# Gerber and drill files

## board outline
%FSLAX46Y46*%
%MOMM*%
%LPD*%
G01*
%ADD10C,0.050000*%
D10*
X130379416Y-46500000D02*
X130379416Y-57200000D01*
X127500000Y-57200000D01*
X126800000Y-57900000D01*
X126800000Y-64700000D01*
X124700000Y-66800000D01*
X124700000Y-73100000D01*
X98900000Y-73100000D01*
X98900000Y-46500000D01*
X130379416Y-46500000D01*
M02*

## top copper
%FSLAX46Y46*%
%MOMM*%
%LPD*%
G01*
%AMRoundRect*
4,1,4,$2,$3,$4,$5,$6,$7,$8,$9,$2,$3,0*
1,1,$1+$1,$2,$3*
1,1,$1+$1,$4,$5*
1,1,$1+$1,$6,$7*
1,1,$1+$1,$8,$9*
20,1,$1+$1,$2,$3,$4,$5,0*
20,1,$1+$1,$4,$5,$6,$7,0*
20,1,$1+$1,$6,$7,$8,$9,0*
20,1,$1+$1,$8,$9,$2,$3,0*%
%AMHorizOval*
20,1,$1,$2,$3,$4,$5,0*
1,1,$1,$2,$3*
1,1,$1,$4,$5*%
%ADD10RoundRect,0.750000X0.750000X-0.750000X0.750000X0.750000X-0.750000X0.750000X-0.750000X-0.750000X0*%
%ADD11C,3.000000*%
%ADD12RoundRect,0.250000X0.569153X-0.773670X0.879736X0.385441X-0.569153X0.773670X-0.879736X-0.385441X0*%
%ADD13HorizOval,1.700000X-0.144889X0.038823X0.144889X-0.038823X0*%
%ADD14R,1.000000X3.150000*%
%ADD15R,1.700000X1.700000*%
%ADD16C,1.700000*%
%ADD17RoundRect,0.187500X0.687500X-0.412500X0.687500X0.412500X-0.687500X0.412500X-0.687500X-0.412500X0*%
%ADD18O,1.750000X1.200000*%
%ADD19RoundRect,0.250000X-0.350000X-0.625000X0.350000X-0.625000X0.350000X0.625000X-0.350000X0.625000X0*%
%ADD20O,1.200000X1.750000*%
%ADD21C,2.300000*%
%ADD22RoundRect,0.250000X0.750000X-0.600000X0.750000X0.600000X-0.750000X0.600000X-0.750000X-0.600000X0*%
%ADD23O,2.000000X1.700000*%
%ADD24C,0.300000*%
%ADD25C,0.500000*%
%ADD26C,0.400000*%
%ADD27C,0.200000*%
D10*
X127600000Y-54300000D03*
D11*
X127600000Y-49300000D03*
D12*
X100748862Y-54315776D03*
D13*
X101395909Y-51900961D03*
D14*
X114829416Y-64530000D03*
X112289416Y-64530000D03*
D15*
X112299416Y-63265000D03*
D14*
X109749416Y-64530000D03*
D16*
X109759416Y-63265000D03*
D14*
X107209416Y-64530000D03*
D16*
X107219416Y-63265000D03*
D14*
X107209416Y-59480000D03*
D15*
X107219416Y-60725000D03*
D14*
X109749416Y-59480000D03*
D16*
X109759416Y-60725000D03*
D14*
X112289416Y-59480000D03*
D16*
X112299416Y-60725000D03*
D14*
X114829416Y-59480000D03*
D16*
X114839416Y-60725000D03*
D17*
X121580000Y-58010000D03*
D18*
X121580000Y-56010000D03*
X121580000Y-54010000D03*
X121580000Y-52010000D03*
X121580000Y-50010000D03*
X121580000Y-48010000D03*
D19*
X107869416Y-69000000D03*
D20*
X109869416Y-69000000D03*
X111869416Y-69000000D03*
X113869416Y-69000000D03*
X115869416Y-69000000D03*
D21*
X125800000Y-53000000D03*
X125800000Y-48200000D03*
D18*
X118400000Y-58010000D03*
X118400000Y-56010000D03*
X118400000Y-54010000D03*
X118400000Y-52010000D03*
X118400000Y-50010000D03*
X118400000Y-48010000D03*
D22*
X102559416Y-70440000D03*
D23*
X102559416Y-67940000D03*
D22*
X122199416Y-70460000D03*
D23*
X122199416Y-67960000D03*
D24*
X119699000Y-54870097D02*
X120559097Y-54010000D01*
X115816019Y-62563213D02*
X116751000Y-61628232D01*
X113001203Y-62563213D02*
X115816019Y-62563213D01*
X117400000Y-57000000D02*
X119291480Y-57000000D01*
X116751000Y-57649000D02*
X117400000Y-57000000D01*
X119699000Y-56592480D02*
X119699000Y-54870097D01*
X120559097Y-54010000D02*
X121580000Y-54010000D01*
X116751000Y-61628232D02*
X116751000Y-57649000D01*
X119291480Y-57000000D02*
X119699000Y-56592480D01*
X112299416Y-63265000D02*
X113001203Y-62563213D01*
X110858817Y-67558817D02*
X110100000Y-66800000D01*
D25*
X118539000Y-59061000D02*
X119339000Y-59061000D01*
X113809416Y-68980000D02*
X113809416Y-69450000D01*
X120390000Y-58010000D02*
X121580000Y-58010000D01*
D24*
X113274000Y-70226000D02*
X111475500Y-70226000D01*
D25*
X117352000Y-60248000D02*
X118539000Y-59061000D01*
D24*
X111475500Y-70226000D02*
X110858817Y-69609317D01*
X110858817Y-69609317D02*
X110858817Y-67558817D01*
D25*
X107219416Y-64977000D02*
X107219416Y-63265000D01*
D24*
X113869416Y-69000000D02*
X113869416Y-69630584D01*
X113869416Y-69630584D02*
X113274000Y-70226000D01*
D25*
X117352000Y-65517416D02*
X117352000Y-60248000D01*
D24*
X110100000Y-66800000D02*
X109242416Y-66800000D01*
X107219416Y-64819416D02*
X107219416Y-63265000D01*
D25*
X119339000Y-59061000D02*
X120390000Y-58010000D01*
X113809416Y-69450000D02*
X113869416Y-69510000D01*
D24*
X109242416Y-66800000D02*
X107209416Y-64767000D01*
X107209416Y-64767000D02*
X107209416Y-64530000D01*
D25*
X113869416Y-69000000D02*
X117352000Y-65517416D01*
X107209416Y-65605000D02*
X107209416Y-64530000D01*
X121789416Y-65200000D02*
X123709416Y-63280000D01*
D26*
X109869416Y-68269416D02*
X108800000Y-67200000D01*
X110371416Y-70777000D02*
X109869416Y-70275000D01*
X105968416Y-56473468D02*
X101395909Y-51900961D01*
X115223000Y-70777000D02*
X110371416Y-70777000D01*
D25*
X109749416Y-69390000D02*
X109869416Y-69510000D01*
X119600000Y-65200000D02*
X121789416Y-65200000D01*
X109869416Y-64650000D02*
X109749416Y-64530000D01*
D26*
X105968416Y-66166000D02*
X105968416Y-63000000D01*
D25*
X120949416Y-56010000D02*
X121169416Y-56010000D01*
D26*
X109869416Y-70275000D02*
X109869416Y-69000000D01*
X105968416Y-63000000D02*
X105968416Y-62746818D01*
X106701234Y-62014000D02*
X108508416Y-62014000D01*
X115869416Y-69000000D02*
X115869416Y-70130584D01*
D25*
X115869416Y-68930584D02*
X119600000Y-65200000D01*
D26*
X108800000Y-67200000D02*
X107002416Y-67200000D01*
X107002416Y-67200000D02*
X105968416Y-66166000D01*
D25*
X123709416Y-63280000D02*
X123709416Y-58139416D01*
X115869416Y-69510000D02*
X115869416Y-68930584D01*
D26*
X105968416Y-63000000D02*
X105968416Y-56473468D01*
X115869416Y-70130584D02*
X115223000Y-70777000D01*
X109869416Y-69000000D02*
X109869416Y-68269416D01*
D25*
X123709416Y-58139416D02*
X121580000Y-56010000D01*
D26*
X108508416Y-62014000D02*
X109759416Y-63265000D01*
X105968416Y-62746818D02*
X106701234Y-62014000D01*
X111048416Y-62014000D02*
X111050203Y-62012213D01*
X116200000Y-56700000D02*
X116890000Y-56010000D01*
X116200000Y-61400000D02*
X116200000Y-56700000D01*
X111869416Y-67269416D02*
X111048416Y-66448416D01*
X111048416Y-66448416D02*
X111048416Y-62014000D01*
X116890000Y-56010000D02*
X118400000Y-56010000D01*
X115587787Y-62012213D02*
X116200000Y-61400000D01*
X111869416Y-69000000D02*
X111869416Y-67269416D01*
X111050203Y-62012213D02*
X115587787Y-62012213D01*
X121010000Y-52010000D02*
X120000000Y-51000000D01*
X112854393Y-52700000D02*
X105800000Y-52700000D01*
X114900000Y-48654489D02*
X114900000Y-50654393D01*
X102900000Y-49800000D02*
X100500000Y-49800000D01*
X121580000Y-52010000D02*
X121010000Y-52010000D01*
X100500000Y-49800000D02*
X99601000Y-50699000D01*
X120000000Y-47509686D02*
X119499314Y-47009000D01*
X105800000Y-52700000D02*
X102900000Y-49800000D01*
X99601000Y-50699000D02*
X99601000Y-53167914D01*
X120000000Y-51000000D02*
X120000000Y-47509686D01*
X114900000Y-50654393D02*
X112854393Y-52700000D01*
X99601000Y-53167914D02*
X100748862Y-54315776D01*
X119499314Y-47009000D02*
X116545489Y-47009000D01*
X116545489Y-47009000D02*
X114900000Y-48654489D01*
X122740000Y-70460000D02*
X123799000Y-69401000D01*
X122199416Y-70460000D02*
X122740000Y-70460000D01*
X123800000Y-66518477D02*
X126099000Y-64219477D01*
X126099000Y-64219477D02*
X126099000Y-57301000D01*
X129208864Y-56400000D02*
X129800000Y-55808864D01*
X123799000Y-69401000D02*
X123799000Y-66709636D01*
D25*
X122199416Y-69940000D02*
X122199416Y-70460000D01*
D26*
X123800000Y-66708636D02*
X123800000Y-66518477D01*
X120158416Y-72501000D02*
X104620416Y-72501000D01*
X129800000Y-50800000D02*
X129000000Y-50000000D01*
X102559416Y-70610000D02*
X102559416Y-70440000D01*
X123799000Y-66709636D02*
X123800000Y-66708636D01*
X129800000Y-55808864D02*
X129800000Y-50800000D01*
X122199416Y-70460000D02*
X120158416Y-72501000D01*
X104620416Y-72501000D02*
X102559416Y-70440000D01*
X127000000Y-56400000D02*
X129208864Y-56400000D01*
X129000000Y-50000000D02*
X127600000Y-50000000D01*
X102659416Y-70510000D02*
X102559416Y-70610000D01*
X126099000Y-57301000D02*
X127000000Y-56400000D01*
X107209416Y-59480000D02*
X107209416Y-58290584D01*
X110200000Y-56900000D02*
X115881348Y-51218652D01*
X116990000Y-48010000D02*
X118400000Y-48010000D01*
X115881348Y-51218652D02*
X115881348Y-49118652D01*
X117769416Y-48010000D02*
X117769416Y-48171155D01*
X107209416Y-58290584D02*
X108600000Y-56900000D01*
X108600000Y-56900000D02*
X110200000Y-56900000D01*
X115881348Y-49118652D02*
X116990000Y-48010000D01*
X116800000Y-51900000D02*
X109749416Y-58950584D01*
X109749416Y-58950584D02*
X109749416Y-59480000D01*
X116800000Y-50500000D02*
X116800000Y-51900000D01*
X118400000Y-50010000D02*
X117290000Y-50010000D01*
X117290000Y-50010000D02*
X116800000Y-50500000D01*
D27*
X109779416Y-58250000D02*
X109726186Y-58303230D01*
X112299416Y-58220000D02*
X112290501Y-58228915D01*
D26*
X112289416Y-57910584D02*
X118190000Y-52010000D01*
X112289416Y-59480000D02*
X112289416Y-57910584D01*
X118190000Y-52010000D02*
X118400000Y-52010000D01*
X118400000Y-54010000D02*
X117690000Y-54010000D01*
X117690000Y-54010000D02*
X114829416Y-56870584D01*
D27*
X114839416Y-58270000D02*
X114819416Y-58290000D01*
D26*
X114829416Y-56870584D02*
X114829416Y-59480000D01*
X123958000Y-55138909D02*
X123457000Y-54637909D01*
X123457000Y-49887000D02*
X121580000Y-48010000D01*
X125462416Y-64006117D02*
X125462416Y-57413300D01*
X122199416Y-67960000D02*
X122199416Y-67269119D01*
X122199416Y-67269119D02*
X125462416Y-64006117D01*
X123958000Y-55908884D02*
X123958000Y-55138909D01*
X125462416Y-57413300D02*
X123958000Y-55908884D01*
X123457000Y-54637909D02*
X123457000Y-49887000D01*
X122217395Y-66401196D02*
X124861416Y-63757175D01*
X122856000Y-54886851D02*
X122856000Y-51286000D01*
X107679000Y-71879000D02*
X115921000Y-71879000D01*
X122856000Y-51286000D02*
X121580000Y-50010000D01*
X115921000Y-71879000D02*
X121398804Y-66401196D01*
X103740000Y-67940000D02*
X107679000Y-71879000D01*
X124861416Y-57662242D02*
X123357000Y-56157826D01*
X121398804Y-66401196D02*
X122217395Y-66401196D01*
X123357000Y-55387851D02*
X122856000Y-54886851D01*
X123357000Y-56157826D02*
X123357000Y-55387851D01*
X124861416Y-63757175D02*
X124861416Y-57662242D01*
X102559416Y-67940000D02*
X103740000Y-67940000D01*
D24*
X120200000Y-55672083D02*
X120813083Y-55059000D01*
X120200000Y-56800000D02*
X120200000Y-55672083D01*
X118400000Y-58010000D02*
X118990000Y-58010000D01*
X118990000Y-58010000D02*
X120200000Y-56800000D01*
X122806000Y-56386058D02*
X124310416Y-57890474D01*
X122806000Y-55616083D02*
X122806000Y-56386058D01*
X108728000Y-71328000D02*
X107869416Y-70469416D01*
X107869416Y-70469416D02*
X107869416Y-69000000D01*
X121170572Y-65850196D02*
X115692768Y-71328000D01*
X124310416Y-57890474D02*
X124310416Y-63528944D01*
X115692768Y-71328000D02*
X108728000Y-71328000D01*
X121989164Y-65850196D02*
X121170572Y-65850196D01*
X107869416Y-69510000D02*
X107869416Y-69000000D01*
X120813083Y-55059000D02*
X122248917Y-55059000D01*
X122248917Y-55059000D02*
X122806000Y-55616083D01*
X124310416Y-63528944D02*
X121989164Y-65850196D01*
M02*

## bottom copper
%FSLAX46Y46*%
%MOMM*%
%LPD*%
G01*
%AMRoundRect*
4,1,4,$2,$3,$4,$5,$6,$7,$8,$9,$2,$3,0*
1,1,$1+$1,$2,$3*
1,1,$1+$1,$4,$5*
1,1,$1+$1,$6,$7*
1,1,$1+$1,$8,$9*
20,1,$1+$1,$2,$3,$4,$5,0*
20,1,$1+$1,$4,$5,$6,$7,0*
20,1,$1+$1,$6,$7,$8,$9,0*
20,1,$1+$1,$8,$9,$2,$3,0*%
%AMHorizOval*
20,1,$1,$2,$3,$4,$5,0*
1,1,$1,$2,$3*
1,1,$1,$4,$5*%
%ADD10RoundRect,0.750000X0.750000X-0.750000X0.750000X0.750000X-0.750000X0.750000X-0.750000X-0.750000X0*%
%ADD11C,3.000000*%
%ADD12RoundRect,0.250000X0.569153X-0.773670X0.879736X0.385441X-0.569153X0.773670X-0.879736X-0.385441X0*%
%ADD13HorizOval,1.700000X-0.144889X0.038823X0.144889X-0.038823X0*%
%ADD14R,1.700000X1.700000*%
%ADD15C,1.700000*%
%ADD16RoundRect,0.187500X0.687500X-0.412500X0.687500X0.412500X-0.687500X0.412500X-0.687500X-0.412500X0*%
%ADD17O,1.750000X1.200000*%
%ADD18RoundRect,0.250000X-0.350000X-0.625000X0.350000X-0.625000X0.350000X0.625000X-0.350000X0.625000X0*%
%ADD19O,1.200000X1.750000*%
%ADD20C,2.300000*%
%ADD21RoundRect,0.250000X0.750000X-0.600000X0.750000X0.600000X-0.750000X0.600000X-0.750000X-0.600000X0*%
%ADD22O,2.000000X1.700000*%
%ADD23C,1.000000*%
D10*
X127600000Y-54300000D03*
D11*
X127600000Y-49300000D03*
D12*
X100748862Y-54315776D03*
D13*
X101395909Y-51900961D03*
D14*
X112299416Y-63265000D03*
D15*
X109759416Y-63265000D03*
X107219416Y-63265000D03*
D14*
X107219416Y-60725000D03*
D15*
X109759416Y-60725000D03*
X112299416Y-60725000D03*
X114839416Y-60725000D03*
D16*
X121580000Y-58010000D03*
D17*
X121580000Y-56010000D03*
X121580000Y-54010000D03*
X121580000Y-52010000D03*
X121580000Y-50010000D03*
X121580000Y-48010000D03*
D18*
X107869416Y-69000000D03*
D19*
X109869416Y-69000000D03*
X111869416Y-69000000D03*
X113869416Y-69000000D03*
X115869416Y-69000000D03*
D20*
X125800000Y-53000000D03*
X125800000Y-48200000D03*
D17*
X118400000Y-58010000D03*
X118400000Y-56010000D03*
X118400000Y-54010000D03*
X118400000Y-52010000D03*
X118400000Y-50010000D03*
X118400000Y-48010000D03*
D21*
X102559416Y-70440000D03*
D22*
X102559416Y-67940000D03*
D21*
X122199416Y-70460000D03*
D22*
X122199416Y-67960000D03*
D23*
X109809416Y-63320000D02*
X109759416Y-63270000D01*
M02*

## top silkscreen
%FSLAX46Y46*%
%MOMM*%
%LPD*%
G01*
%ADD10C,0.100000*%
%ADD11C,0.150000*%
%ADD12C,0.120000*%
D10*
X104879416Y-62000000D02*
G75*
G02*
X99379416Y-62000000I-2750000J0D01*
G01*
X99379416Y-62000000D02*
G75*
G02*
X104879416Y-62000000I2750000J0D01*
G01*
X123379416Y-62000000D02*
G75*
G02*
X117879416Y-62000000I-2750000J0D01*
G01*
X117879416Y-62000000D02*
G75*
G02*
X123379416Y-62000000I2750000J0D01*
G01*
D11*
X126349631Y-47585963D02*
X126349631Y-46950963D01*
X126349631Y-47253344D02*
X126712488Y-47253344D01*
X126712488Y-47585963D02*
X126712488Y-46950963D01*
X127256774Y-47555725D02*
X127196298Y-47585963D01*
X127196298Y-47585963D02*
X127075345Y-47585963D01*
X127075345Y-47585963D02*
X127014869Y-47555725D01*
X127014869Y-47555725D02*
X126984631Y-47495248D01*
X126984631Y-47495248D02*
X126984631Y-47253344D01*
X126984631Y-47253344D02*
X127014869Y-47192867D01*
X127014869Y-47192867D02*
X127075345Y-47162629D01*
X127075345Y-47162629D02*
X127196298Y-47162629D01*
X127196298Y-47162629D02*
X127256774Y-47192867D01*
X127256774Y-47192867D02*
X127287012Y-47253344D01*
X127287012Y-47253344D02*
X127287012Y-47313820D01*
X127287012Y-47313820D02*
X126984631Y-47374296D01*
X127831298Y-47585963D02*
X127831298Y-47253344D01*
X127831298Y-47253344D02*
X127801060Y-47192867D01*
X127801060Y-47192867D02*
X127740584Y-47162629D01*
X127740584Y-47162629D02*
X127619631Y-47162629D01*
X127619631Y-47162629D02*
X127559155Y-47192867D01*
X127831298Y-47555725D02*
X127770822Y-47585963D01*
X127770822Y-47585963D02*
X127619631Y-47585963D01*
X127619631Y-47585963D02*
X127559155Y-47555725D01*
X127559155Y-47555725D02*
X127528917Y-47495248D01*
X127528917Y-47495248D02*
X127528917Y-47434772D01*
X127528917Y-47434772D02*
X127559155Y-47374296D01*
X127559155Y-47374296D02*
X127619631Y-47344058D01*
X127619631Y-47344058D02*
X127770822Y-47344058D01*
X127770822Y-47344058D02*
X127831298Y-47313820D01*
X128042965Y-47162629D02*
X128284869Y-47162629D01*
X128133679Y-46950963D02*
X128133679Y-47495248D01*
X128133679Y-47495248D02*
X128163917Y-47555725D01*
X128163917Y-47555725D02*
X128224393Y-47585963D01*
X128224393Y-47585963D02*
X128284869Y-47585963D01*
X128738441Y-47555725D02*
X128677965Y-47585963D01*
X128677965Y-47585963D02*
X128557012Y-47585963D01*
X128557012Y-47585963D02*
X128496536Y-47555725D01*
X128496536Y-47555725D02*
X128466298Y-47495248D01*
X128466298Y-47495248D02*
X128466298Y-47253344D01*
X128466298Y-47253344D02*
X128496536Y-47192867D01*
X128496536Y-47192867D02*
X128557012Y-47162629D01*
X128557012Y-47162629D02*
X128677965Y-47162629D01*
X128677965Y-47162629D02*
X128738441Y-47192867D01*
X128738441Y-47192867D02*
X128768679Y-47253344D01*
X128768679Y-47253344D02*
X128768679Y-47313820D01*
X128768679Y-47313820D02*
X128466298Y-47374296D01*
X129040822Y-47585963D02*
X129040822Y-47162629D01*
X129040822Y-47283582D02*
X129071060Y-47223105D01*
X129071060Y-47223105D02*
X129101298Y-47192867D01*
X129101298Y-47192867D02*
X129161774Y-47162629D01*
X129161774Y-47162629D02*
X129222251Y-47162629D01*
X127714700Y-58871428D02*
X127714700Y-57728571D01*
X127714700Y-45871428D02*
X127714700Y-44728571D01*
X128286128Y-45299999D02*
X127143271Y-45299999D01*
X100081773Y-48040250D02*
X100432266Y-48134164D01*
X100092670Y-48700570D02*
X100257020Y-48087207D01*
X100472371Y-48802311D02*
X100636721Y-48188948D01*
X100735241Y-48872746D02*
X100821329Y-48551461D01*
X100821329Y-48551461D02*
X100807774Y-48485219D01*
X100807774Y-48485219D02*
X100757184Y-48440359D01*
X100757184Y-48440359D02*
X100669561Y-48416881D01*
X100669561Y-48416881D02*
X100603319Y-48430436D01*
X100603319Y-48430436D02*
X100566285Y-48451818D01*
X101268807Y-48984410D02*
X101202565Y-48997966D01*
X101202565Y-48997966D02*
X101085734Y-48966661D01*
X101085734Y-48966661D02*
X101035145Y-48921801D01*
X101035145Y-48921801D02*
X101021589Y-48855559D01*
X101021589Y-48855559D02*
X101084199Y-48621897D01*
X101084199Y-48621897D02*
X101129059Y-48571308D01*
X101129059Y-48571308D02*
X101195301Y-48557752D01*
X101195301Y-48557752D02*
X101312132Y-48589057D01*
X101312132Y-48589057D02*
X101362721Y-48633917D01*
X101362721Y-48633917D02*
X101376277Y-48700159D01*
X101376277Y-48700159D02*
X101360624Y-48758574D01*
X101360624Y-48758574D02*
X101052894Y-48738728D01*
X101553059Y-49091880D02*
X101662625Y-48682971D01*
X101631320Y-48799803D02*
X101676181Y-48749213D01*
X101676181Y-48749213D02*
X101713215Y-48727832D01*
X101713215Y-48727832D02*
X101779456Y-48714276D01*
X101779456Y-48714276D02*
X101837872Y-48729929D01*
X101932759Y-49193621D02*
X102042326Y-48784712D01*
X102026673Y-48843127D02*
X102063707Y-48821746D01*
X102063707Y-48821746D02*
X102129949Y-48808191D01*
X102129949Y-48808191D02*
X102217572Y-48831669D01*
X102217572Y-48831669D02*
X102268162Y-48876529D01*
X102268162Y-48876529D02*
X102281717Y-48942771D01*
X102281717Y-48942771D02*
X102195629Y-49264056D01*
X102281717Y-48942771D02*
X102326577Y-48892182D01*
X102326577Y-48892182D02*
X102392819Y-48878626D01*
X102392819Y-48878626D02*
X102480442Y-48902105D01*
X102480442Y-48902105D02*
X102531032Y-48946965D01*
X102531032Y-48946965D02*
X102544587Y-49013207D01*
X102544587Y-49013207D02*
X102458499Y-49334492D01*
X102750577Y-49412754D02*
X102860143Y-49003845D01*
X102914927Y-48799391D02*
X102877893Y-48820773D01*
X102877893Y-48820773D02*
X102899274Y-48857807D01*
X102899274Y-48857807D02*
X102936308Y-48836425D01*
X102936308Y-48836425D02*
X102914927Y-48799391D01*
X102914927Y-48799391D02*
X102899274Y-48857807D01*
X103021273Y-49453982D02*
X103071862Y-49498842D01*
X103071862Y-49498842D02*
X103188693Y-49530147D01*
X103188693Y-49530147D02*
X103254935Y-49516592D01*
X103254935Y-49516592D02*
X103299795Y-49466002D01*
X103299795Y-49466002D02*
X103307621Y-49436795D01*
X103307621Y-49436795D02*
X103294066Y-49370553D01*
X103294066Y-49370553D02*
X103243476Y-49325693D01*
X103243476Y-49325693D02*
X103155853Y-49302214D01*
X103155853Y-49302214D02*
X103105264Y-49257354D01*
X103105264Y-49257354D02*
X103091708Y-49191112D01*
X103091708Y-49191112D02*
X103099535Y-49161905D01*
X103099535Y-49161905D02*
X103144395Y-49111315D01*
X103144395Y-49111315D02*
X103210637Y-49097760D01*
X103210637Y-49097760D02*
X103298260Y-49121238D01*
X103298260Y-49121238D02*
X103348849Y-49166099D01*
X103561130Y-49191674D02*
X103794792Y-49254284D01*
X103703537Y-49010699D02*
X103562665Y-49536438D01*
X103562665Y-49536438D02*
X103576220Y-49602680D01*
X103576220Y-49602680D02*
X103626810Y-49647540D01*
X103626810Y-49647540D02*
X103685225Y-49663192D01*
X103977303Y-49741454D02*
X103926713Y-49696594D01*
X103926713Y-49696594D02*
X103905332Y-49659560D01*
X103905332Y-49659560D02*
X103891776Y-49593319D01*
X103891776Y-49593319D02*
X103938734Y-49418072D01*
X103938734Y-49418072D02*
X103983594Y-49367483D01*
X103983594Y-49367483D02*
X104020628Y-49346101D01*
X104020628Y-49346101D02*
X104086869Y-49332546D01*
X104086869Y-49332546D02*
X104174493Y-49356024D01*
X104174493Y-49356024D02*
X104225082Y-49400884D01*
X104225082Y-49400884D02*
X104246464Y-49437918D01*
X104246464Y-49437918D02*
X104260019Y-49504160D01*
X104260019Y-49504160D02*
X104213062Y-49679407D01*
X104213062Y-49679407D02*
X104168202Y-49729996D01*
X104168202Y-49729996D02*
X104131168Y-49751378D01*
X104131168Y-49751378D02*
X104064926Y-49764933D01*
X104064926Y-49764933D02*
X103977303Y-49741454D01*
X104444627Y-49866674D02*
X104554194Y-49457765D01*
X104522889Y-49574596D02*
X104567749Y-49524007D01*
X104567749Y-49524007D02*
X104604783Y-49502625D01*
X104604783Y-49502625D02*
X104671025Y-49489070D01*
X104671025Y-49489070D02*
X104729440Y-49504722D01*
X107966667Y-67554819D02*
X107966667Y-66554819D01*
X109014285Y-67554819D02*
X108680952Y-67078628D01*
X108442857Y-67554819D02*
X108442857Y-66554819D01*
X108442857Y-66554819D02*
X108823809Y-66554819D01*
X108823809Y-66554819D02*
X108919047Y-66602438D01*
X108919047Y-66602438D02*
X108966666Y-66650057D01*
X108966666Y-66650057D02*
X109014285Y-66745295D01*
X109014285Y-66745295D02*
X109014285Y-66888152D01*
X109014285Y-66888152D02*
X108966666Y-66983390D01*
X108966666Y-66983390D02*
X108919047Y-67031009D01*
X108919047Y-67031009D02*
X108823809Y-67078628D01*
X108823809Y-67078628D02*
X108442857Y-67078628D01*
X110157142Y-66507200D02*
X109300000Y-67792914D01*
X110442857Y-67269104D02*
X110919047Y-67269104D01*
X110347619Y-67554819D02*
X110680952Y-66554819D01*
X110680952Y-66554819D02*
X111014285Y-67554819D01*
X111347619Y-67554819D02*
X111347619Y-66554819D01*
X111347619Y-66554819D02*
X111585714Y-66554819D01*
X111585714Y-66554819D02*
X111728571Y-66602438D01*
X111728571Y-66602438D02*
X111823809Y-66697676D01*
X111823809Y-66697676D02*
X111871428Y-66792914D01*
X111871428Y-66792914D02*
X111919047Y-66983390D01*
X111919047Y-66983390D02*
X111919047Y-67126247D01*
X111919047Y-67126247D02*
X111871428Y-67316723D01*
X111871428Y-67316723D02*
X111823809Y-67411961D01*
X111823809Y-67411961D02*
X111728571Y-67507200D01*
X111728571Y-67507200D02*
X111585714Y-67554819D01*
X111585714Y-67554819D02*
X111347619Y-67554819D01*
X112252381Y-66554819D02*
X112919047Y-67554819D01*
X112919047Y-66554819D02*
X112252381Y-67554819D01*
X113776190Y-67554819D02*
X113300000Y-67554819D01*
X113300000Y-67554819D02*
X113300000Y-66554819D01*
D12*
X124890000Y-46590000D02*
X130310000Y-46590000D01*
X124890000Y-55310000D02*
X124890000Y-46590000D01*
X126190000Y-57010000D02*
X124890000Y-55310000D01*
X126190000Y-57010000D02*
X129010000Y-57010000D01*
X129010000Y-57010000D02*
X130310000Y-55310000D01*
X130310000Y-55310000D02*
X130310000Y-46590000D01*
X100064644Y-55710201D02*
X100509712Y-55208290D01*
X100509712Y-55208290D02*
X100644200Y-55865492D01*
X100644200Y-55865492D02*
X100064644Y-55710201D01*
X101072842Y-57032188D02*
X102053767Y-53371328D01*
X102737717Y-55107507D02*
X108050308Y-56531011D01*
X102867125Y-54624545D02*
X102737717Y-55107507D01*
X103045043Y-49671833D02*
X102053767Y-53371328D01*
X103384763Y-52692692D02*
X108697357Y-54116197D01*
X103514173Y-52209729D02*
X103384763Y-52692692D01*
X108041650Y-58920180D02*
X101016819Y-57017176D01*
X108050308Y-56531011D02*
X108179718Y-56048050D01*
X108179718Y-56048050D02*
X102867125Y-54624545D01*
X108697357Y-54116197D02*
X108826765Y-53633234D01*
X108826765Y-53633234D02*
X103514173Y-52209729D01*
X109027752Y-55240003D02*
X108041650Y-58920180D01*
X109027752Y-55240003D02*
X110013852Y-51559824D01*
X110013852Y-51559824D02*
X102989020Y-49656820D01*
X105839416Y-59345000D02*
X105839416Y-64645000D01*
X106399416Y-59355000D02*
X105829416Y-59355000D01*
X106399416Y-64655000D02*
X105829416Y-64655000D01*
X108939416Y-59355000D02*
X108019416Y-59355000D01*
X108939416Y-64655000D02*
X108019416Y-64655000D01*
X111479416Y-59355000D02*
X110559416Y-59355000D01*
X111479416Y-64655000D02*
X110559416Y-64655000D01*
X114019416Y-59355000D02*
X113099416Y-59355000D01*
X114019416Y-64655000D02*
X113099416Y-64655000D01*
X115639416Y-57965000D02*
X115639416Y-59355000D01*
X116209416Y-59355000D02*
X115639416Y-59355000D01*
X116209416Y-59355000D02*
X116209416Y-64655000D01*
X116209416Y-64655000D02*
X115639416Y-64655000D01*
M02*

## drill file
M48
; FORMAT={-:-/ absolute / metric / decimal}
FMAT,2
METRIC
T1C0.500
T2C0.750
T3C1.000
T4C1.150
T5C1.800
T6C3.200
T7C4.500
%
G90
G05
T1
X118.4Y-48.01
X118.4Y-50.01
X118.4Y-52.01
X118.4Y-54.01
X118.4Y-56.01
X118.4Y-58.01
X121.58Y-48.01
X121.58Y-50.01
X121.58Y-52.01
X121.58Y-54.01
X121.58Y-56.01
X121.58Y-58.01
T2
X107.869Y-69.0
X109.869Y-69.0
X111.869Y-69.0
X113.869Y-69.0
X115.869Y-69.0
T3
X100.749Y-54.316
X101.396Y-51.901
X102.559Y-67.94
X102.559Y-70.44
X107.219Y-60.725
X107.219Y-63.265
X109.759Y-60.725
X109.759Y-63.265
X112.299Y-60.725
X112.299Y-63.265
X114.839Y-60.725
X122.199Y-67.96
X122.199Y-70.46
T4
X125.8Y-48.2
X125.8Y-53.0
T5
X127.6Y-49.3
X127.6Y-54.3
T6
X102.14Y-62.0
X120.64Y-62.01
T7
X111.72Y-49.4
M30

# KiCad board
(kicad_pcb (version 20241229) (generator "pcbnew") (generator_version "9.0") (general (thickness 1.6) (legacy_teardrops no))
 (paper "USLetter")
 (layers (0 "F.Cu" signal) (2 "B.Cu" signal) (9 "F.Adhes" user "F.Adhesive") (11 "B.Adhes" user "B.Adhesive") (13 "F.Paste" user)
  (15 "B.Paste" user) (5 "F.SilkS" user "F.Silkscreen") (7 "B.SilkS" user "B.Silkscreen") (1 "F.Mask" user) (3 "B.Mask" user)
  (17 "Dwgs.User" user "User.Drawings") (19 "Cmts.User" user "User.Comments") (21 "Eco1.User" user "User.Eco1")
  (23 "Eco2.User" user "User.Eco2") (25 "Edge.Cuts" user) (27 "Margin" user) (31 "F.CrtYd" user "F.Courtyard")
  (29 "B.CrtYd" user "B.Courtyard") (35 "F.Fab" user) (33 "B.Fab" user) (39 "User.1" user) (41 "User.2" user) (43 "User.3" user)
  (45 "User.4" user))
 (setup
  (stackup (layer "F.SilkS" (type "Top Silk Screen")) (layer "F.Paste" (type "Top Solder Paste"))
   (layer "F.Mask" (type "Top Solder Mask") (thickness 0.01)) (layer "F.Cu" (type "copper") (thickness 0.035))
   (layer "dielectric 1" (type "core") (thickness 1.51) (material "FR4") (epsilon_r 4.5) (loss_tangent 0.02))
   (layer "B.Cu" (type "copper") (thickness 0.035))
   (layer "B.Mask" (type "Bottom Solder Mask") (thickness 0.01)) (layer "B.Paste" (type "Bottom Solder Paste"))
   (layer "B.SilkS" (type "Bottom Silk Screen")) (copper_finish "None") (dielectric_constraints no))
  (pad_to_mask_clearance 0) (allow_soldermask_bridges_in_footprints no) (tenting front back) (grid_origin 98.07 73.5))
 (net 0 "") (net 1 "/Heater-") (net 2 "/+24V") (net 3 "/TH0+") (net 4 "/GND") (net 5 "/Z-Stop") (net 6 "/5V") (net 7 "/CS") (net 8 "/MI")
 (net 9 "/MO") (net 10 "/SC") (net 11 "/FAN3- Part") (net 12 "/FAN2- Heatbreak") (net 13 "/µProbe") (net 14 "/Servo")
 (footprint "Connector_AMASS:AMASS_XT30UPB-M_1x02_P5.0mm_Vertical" (layer "F.Cu") (at 127.6 54.3 90)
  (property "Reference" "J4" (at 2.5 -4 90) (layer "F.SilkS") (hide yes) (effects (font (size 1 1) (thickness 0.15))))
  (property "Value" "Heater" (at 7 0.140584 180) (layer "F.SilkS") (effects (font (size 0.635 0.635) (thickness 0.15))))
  (fp_line (start 7.71 -2.71) (end 7.71 2.71) (stroke (width 0.12) (type solid)) (layer "F.SilkS"))
  (fp_line (start -1.01 -2.71) (end 7.71 -2.71) (stroke (width 0.12) (type solid)) (layer "F.SilkS"))
  (fp_line (start -2.71 -1.41) (end -1.01 -2.71) (stroke (width 0.12) (type solid)) (layer "F.SilkS"))
  (fp_line (start -2.71 -1.41) (end -2.71 1.41) (stroke (width 0.12) (type solid)) (layer "F.SilkS"))
  (fp_line (start -2.71 1.41) (end -1.01 2.71) (stroke (width 0.12) (type solid)) (layer "F.SilkS"))
  (fp_line (start -1.01 2.71) (end 7.71 2.71) (stroke (width 0.12) (type solid)) (layer "F.SilkS"))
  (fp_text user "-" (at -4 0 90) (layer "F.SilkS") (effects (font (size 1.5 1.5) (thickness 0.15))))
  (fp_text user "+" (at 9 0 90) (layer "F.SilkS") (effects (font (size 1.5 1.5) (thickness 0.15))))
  (pad "1" thru_hole roundrect (at 0 0 90) (size 3 3) (drill 1.8) (layers "*.Cu" "*.Mask") (remove_unused_layers no) (roundrect_rratio 0.25)
   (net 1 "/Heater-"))
  (pad "2" thru_hole circle (at 5 0 90) (size 3 3) (drill 1.8) (layers "*.Cu" "*.Mask") (remove_unused_layers no) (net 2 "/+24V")))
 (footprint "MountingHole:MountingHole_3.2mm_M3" (layer "F.Cu") (at 120.64 62.01)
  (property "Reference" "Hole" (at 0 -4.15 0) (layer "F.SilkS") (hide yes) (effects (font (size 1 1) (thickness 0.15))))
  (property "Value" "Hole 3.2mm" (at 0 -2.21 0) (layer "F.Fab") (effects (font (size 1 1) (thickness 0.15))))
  (pad "" np_thru_hole circle (at 0 0) (size 3.2 3.2) (drill 3.2) (layers "*.Cu" "*.Mask")))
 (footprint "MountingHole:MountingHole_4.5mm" (layer "F.Cu") (at 111.72 49.4)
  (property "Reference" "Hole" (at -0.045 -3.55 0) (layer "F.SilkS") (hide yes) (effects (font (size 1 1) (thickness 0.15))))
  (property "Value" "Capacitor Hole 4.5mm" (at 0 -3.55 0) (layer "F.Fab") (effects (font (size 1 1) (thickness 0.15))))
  (pad "" np_thru_hole circle (at 0 0) (size 4.5 4.5) (drill 4.5) (layers "*.Cu" "*.Mask")))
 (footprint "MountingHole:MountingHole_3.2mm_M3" (layer "F.Cu") (at 102.14 62)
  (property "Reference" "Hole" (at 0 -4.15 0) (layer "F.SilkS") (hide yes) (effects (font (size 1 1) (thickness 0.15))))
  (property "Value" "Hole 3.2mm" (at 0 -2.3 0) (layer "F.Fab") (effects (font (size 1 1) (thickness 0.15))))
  (pad "" np_thru_hole circle (at 0 0) (size 3.2 3.2) (drill 3.2) (layers "*.Cu" "*.Mask")))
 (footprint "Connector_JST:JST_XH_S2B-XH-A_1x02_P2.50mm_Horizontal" (layer "F.Cu") (at 100.748862 54.315776 75)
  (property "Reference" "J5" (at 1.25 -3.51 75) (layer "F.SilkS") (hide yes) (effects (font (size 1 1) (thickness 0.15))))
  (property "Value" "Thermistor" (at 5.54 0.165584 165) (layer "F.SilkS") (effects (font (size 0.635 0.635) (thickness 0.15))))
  (fp_line (start -1.524 -0.3) (end -0.923999 -0.000002) (stroke (width 0.12) (type solid)) (layer "F.SilkS"))
  (fp_line (start -0.923999 -0.000002) (end -1.523999 0.3) (stroke (width 0.12) (type solid)) (layer "F.SilkS"))
  (fp_line (start -1.523999 0.3) (end -1.524 -0.3) (stroke (width 0.12) (type solid)) (layer "F.SilkS"))
  (fp_line (start -2.54 1.016) (end 1.250001 1.016) (stroke (width 0.12) (type solid)) (layer "F.SilkS"))
  (fp_line (start -0.25 2.126001) (end -0.249999 7.626) (stroke (width 0.12) (type solid)) (layer "F.SilkS"))
  (fp_line (start 0.249999 2.126) (end -0.25 2.126001) (stroke (width 0.12) (type solid)) (layer "F.SilkS"))
  (fp_line (start 5.08 1.016) (end 1.250001 1.016) (stroke (width 0.12) (type solid)) (layer "F.SilkS"))
  (fp_line (start 2.25 2.126) (end 2.25 7.626002) (stroke (width 0.12) (type solid)) (layer "F.SilkS"))
  (fp_line (start 2.75 2.126) (end 2.25 2.126) (stroke (width 0.12) (type solid)) (layer "F.SilkS"))
  (fp_line (start -2.56 8.236) (end -2.54 0.958) (stroke (width 0.12) (type solid)) (layer "F.SilkS"))
  (fp_line (start -0.249999 7.626) (end 0.249999 7.626001) (stroke (width 0.12) (type solid)) (layer "F.SilkS"))
  (fp_line (start 0.249999 7.626001) (end 0.249999 2.126) (stroke (width 0.12) (type solid)) (layer "F.SilkS"))
  (fp_line (start 2.25 7.626002) (end 2.75 7.626) (stroke (width 0.12) (type solid)) (layer "F.SilkS"))
  (fp_line (start 2.75 7.626) (end 2.75 2.126) (stroke (width 0.12) (type solid)) (layer "F.SilkS"))
  (fp_line (start 1.25 8.236001) (end -2.56 8.236) (stroke (width 0.12) (type solid)) (layer "F.SilkS"))
  (fp_line (start 1.25 8.236001) (end 5.060001 8.236) (stroke (width 0.12) (type solid)) (layer "F.SilkS"))
  (fp_line (start 5.060001 8.236) (end 5.080001 0.958) (stroke (width 0.12) (type solid)) (layer "F.SilkS"))
  (pad "1" thru_hole roundrect (at 0 0 75) (size 1.7 2) (drill 1) (layers "*.Cu" "*.Mask") (remove_unused_layers no)
   (roundrect_rratio 0.147059) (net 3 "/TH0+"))
  (pad "2" thru_hole oval (at 2.5 -0.000001 75) (size 1.7 2) (drill 1) (layers "*.Cu" "*.Mask") (remove_unused_layers no) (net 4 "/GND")))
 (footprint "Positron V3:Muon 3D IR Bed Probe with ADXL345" (layer "F.Cu") (at 109.339416 58.225)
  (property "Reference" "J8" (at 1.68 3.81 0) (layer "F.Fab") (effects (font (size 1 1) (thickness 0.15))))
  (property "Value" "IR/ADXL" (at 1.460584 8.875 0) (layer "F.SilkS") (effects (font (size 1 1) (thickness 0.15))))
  (fp_line (start -3.5 1.12) (end -3.5 6.42) (stroke (width 0.12) (type solid)) (layer "F.SilkS"))
  (fp_line (start -2.94 1.13) (end -3.51 1.13) (stroke (width 0.12) (type solid)) (layer "F.SilkS"))
  (fp_line (start -2.94 6.43) (end -3.51 6.43) (stroke (width 0.12) (type solid)) (layer "F.SilkS"))
  (fp_line (start -0.4 1.13) (end -1.32 1.13) (stroke (width 0.12) (type solid)) (layer "F.SilkS"))
  (fp_line (start -0.4 6.43) (end -1.32 6.43) (stroke (width 0.12) (type solid)) (layer "F.SilkS"))
  (fp_line (start 2.14 1.13) (end 1.22 1.13) (stroke (width 0.12) (type solid)) (layer "F.SilkS"))
  (fp_line (start 2.14 6.43) (end 1.22 6.43) (stroke (width 0.12) (type solid)) (layer "F.SilkS"))
  (fp_line (start 4.68 1.13) (end 3.76 1.13) (stroke (width 0.12) (type solid)) (layer "F.SilkS"))
  (fp_line (start 4.68 6.43) (end 3.76 6.43) (stroke (width 0.12) (type solid)) (layer "F.SilkS"))
  (fp_line (start 6.3 -0.26) (end 6.3 1.13) (stroke (width 0.12) (type solid)) (layer "F.SilkS"))
  (fp_line (start 6.87 1.13) (end 6.3 1.13) (stroke (width 0.12) (type solid)) (layer "F.SilkS"))
  (fp_line (start 6.87 1.13) (end 6.87 6.43) (stroke (width 0.12) (type solid)) (layer "F.SilkS"))
  (fp_line (start 6.87 6.43) (end 6.3 6.43) (stroke (width 0.12) (type solid)) (layer "F.SilkS"))
  (pad "" smd rect (at 5.49 6.305 270) (size 3.15 1) (layers "F.Cu" "F.Mask" "F.Paste"))
  (pad "1" smd rect (at 2.95 6.305 270) (size 3.15 1) (layers "F.Cu" "F.Mask" "F.Paste") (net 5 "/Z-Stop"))
  (pad "1" thru_hole rect (at 2.96 5.04 270) (size 1.7 1.7) (drill 1) (layers "*.Cu" "*.Mask") (remove_unused_layers no) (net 5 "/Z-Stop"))
  (pad "2" smd rect (at 0.41 6.305 270) (size 3.15 1) (layers "F.Cu" "F.Mask" "F.Paste") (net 4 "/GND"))
  (pad "2" thru_hole circle (at 0.42 5.04 270) (size 1.7 1.7) (drill 1) (layers "*.Cu" "*.Mask") (remove_unused_layers no) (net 4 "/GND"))
  (pad "3" smd rect (at -2.13 6.305 270) (size 3.15 1) (layers "F.Cu" "F.Mask" "F.Paste") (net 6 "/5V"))
  (pad "3" thru_hole circle (at -2.12 5.04 270) (size 1.7 1.7) (drill 1) (layers "*.Cu" "*.Mask") (remove_unused_layers no) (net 6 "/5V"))
  (pad "4" smd rect (at -2.13 1.255 270) (size 3.15 1) (layers "F.Cu" "F.Mask" "F.Paste") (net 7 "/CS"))
  (pad "4" thru_hole rect (at -2.12 2.5 270) (size 1.7 1.7) (drill 1) (layers "*.Cu" "*.Mask") (remove_unused_layers no) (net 7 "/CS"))
  (pad "5" smd rect (at 0.41 1.255 270) (size 3.15 1) (layers "F.Cu" "F.Mask" "F.Paste") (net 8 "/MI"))
  (pad "5" thru_hole circle (at 0.42 2.5 270) (size 1.7 1.7) (drill 1) (layers "*.Cu" "*.Mask") (remove_unused_layers no) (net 8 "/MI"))
  (pad "6" smd rect (at 2.95 1.255 270) (size 3.15 1) (layers "F.Cu" "F.Mask" "F.Paste") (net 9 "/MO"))
  (pad "6" thru_hole circle (at 2.96 2.5 270) (size 1.7 1.7) (drill 1) (layers "*.Cu" "*.Mask") (remove_unused_layers no) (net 9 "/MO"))
  (pad "7" smd rect (at 5.49 1.255 270) (size 3.15 1) (layers "F.Cu" "F.Mask" "F.Paste") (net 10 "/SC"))
  (pad "7" thru_hole circle (at 5.5 2.5 270) (size 1.7 1.7) (drill 1) (layers "*.Cu" "*.Mask") (remove_unused_layers no) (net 10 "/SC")))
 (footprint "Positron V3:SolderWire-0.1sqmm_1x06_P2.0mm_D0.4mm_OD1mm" (layer "B.Cu") (at 121.58 58.01 90)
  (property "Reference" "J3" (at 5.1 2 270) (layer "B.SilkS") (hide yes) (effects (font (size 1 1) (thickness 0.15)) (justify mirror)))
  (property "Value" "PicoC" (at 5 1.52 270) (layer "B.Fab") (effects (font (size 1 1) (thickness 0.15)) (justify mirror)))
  (pad "1" thru_hole roundrect (at 0 0 90) (size 1.2 1.75) (drill 0.5) (layers "*.Cu" "*.Mask") (remove_unused_layers no)
   (roundrect_rratio 0.15625) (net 6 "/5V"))
  (pad "2" thru_hole oval (at 2 0 90) (size 1.2 1.75) (drill 0.5) (layers "*.Cu" "*.Mask") (remove_unused_layers no) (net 4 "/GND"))
  (pad "3" thru_hole oval (at 4 0 90) (size 1.2 1.75) (drill 0.5) (layers "*.Cu" "*.Mask") (remove_unused_layers no) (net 5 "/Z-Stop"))
  (pad "4" thru_hole oval (at 6 0 90) (size 1.2 1.75) (drill 0.5) (layers "*.Cu" "*.Mask") (remove_unused_layers no) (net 3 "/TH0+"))
  (pad "5" thru_hole oval (at 8 0 90) (size 1.2 1.75) (drill 0.5) (layers "*.Cu" "*.Mask") (remove_unused_layers no) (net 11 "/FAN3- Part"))
  (pad "6" thru_hole oval (at 10 0 90) (size 1.2 1.75) (drill 0.5) (layers "*.Cu" "*.Mask") (remove_unused_layers no)
   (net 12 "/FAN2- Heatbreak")))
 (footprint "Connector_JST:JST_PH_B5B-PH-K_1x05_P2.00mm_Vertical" (layer "B.Cu") (at 107.869416 69)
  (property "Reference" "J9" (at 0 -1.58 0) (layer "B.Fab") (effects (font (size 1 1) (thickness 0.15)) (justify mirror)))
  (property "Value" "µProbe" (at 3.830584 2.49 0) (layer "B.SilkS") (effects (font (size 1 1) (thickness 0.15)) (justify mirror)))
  (pad "1" thru_hole roundrect (at 0 0) (size 1.2 1.75) (drill 0.75) (layers "*.Cu" "*.Mask") (remove_unused_layers no)
   (roundrect_rratio 0.208333) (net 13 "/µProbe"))
  (pad "2" thru_hole oval (at 2 0) (size 1.2 1.75) (drill 0.75) (layers "*.Cu" "*.Mask") (remove_unused_layers no) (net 4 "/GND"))
  (pad "3" thru_hole oval (at 4 0) (size 1.2 1.75) (drill 0.75) (layers "*.Cu" "*.Mask") (remove_unused_layers no) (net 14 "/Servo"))
  (pad "4" thru_hole oval (at 6 0) (size 1.2 1.75) (drill 0.75) (layers "*.Cu" "*.Mask") (remove_unused_layers no) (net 6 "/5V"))
  (pad "5" thru_hole oval (at 8 0) (size 1.2 1.75) (drill 0.75) (layers "*.Cu" "*.Mask") (remove_unused_layers no) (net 4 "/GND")))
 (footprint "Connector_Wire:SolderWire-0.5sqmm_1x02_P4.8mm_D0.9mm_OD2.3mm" (layer "B.Cu") (at 125.8 53 90)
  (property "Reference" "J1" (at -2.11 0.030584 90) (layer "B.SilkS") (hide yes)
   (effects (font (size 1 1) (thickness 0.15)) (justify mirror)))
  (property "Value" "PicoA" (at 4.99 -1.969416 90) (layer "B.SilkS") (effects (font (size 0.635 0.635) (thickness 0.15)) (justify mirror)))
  (pad "1" thru_hole circle (at 0 0 90) (size 2.3 2.3) (drill 1.15) (layers "*.Cu" "*.Mask") (remove_unused_layers no) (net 1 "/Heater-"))
  (pad "2" thru_hole circle (at 4.8 0 90) (size 2.3 2.3) (drill 1.15) (layers "*.Cu" "*.Mask") (remove_unused_layers no) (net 2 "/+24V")))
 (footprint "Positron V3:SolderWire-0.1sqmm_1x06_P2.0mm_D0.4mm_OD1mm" (layer "B.Cu") (at 118.4 58.01 90)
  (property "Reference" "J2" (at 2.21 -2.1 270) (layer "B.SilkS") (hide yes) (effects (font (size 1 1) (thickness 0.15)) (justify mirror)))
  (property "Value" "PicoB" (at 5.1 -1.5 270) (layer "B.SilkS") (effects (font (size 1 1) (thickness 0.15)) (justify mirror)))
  (pad "1" thru_hole oval (at 0 0 90) (size 1.2 1.75) (drill 0.5) (layers "*.Cu" "*.Mask") (remove_unused_layers no) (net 13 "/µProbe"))
  (pad "2" thru_hole oval (at 2 0 90) (size 1.2 1.75) (drill 0.5) (layers "*.Cu" "*.Mask") (remove_unused_layers no) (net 14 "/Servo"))
  (pad "3" thru_hole oval (at 4 0 90) (size 1.2 1.75) (drill 0.5) (layers "*.Cu" "*.Mask") (remove_unused_layers no) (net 10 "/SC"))
  (pad "4" thru_hole oval (at 6 0 90) (size 1.2 1.75) (drill 0.5) (layers "*.Cu" "*.Mask") (remove_unused_layers no) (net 9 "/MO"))
  (pad "5" thru_hole oval (at 8 0 90) (size 1.2 1.75) (drill 0.5) (layers "*.Cu" "*.Mask") (remove_unused_layers no) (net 8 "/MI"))
  (pad "6" thru_hole oval (at 10 0 90) (size 1.2 1.75) (drill 0.5) (layers "*.Cu" "*.Mask") (remove_unused_layers no) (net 7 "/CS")))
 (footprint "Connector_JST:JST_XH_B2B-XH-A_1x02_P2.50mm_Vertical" (layer "B.Cu") (at 102.559416 70.44 90)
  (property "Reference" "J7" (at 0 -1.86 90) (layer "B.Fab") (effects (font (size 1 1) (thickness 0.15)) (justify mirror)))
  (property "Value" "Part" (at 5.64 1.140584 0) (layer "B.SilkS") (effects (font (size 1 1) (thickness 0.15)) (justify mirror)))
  (pad "1" thru_hole roundrect (at 0 0 90) (size 1.7 2) (drill 1) (layers "*.Cu" "*.Mask") (remove_unused_layers no)
   (roundrect_rratio 0.147059) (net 2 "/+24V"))
  (pad "2" thru_hole oval (at 2.5 0 90) (size 1.7 2) (drill 1) (layers "*.Cu" "*.Mask") (remove_unused_layers no) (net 11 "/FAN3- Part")))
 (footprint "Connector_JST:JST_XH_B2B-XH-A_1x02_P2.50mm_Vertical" (layer "B.Cu") (at 122.199416 70.46 90)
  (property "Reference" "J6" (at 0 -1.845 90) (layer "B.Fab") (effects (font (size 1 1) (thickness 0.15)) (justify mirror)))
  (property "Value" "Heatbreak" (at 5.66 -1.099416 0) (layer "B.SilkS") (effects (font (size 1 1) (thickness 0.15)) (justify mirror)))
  (pad "1" thru_hole roundrect (at 0 0 90) (size 1.7 2) (drill 1) (layers "*.Cu" "*.Mask") (remove_unused_layers no)
   (roundrect_rratio 0.147059) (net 2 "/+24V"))
  (pad "2" thru_hole oval (at 2.5 0 90) (size 1.7 2) (drill 1) (layers "*.Cu" "*.Mask") (remove_unused_layers no)
   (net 12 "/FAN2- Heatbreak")))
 (gr_circle (center 102.129416 62) (end 104.879416 62) (stroke (width 0.1) (type solid)) (fill no) (layer "F.SilkS"))
 (gr_circle (center 120.629416 62) (end 123.379416 62) (stroke (width 0.1) (type solid)) (fill no) (layer "F.SilkS"))
 (gr_poly
  (pts (xy 130.379416 46.5) (xy 130.379416 57.2) (xy 127.5 57.2) (xy 126.8 57.9) (xy 126.8 64.7) (xy 124.7 66.8) (xy 124.7 73.1)
   (xy 98.9 73.1) (xy 98.9 46.5))
  (stroke (width 0.05) (type solid)) (fill no) (layer "Edge.Cuts"))
 (segment (start 119.699 54.870097) (end 120.559097 54.01) (width 0.3) (layer "F.Cu") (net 5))
 (segment (start 115.816019 62.563213) (end 116.751 61.628232) (width 0.3) (layer "F.Cu") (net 5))
 (segment (start 113.001203 62.563213) (end 115.816019 62.563213) (width 0.3) (layer "F.Cu") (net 5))
 (segment (start 117.4 57) (end 119.29148 57) (width 0.3) (layer "F.Cu") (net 5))
 (segment (start 116.751 57.649) (end 117.4 57) (width 0.3) (layer "F.Cu") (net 5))
 (segment (start 119.699 56.59248) (end 119.699 54.870097) (width 0.3) (layer "F.Cu") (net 5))
 (segment (start 120.559097 54.01) (end 121.58 54.01) (width 0.3) (layer "F.Cu") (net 5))
 (segment (start 116.751 61.628232) (end 116.751 57.649) (width 0.3) (layer "F.Cu") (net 5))
 (segment (start 119.29148 57) (end 119.699 56.59248) (width 0.3) (layer "F.Cu") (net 5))
 (segment (start 112.299416 63.265) (end 113.001203 62.563213) (width 0.3) (layer "F.Cu") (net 5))
 (segment (start 110.858817 67.558817) (end 110.1 66.8) (width 0.3) (layer "F.Cu") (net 6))
 (segment (start 118.539 59.061) (end 119.339 59.061) (width 0.5) (layer "F.Cu") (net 6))
 (segment (start 113.809416 68.98) (end 113.809416 69.45) (width 0.5) (layer "F.Cu") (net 6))
 (segment (start 120.39 58.01) (end 121.58 58.01) (width 0.5) (layer "F.Cu") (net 6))
 (segment (start 113.274 70.226) (end 111.4755 70.226) (width 0.3) (layer "F.Cu") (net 6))
 (segment (start 117.352 60.248) (end 118.539 59.061) (width 0.5) (layer "F.Cu") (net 6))
 (segment (start 111.4755 70.226) (end 110.858817 69.609317) (width 0.3) (layer "F.Cu") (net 6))
 (segment (start 110.858817 69.609317) (end 110.858817 67.558817) (width 0.3) (layer "F.Cu") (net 6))
 (segment (start 107.219416 64.977) (end 107.219416 63.265) (width 0.5) (layer "F.Cu") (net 6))
 (segment (start 113.869416 69) (end 113.869416 69.630584) (width 0.3) (layer "F.Cu") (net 6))
 (segment (start 113.869416 69.630584) (end 113.274 70.226) (width 0.3) (layer "F.Cu") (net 6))
 (segment (start 117.352 65.517416) (end 117.352 60.248) (width 0.5) (layer "F.Cu") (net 6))
 (segment (start 110.1 66.8) (end 109.242416 66.8) (width 0.3) (layer "F.Cu") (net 6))
 (segment (start 107.219416 64.819416) (end 107.219416 63.265) (width 0.3) (layer "F.Cu") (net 6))
 (segment (start 119.339 59.061) (end 120.39 58.01) (width 0.5) (layer "F.Cu") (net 6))
 (segment (start 113.809416 69.45) (end 113.869416 69.51) (width 0.5) (layer "F.Cu") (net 6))
 (segment (start 109.242416 66.8) (end 107.209416 64.767) (width 0.3) (layer "F.Cu") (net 6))
 (segment (start 107.209416 64.767) (end 107.209416 64.53) (width 0.3) (layer "F.Cu") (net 6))
 (segment (start 113.869416 69) (end 117.352 65.517416) (width 0.5) (layer "F.Cu") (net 6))
 (segment (start 107.209416 65.605) (end 107.209416 64.53) (width 0.5) (layer "F.Cu") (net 6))
 (segment (start 121.789416 65.2) (end 123.709416 63.28) (width 0.5) (layer "F.Cu") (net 4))
 (segment (start 109.869416 68.269416) (end 108.8 67.2) (width 0.4) (layer "F.Cu") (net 4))
 (segment (start 110.371416 70.777) (end 109.869416 70.275) (width 0.4) (layer "F.Cu") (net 4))
 (segment (start 105.968416 56.473468) (end 101.395909 51.900961) (width 0.4) (layer "F.Cu") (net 4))
 (segment (start 115.223 70.777) (end 110.371416 70.777) (width 0.4) (layer "F.Cu") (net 4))
 (segment (start 109.749416 69.39) (end 109.869416 69.51) (width 0.5) (layer "F.Cu") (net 4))
 (segment (start 119.6 65.2) (end 121.789416 65.2) (width 0.5) (layer "F.Cu") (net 4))
 (segment (start 109.869416 64.65) (end 109.749416 64.53) (width 0.5) (layer "F.Cu") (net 4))
 (segment (start 105.968416 66.166) (end 105.968416 63) (width 0.4) (layer "F.Cu") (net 4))
 (segment (start 120.949416 56.01) (end 121.169416 56.01) (width 0.5) (layer "F.Cu") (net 4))
 (segment (start 109.869416 70.275) (end 109.869416 69) (width 0.4) (layer "F.Cu") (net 4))
 (segment (start 105.968416 63) (end 105.968416 62.746818) (width 0.4) (layer "F.Cu") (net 4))
 (segment (start 106.701234 62.014) (end 108.508416 62.014) (width 0.4) (layer "F.Cu") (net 4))
 (segment (start 115.869416 69) (end 115.869416 70.130584) (width 0.4) (layer "F.Cu") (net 4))
 (segment (start 115.869416 68.930584) (end 119.6 65.2) (width 0.5) (layer "F.Cu") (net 4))
 (segment (start 108.8 67.2) (end 107.002416 67.2) (width 0.4) (layer "F.Cu") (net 4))
 (segment (start 107.002416 67.2) (end 105.968416 66.166) (width 0.4) (layer "F.Cu") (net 4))
 (segment (start 123.709416 63.28) (end 123.709416 58.139416) (width 0.5) (layer "F.Cu") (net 4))
 (segment (start 115.869416 69.51) (end 115.869416 68.930584) (width 0.5) (layer "F.Cu") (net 4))
 (segment (start 105.968416 63) (end 105.968416 56.473468) (width 0.4) (layer "F.Cu") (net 4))
 (segment (start 115.869416 70.130584) (end 115.223 70.777) (width 0.4) (layer "F.Cu") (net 4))
 (segment (start 109.869416 69) (end 109.869416 68.269416) (width 0.4) (layer "F.Cu") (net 4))
 (segment (start 123.709416 58.139416) (end 121.58 56.01) (width 0.5) (layer "F.Cu") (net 4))
 (segment (start 108.508416 62.014) (end 109.759416 63.265) (width 0.4) (layer "F.Cu") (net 4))
 (segment (start 105.968416 62.746818) (end 106.701234 62.014) (width 0.4) (layer "F.Cu") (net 4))
 (segment (start 109.809416 63.32) (end 109.759416 63.27) (width 1) (layer "B.Cu") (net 4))
 (segment (start 111.048416 62.014) (end 111.050203 62.012213) (width 0.4) (layer "F.Cu") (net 14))
 (segment (start 116.2 56.7) (end 116.89 56.01) (width 0.4) (layer "F.Cu") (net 14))
 (segment (start 116.2 61.4) (end 116.2 56.7) (width 0.4) (layer "F.Cu") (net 14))
 (segment (start 111.869416 67.269416) (end 111.048416 66.448416) (width 0.4) (layer "F.Cu") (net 14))
 (segment (start 111.048416 66.448416) (end 111.048416 62.014) (width 0.4) (layer "F.Cu") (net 14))
 (segment (start 116.89 56.01) (end 118.4 56.01) (width 0.4) (layer "F.Cu") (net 14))
 (segment (start 115.587787 62.012213) (end 116.2 61.4) (width 0.4) (layer "F.Cu") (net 14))
 (segment (start 111.869416 69) (end 111.869416 67.269416) (width 0.4) (layer "F.Cu") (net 14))
 (segment (start 111.050203 62.012213) (end 115.587787 62.012213) (width 0.4) (layer "F.Cu") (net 14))
 (segment (start 121.01 52.01) (end 120 51) (width 0.4) (layer "F.Cu") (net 3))
 (segment (start 112.854393 52.7) (end 105.8 52.7) (width 0.4) (layer "F.Cu") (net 3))
 (segment (start 114.9 48.654489) (end 114.9 50.654393) (width 0.4) (layer "F.Cu") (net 3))
 (segment (start 102.9 49.8) (end 100.5 49.8) (width 0.4) (layer "F.Cu") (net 3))
 (segment (start 121.58 52.01) (end 121.01 52.01) (width 0.4) (layer "F.Cu") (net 3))
 (segment (start 100.5 49.8) (end 99.601 50.699) (width 0.4) (layer "F.Cu") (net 3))
 (segment (start 120 47.509686) (end 119.499314 47.009) (width 0.4) (layer "F.Cu") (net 3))
 (segment (start 105.8 52.7) (end 102.9 49.8) (width 0.4) (layer "F.Cu") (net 3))
 (segment (start 99.601 50.699) (end 99.601 53.167914) (width 0.4) (layer "F.Cu") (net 3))
 (segment (start 120 51) (end 120 47.509686) (width 0.4) (layer "F.Cu") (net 3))
 (segment (start 114.9 50.654393) (end 112.854393 52.7) (width 0.4) (layer "F.Cu") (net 3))
 (segment (start 99.601 53.167914) (end 100.748862 54.315776) (width 0.4) (layer "F.Cu") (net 3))
 (segment (start 119.499314 47.009) (end 116.545489 47.009) (width 0.4) (layer "F.Cu") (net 3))
 (segment (start 116.545489 47.009) (end 114.9 48.654489) (width 0.4) (layer "F.Cu") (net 3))
 (segment (start 122.74 70.46) (end 123.799 69.401) (width 0.4) (layer "F.Cu") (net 2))
 (segment (start 122.199416 70.46) (end 122.74 70.46) (width 0.4) (layer "F.Cu") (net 2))
 (segment (start 123.8 66.518477) (end 126.099 64.219477) (width 0.4) (layer "F.Cu") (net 2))
 (segment (start 126.099 64.219477) (end 126.099 57.301) (width 0.4) (layer "F.Cu") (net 2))
 (segment (start 129.208864 56.4) (end 129.8 55.808864) (width 0.4) (layer "F.Cu") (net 2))
 (segment (start 123.799 69.401) (end 123.799 66.709636) (width 0.4) (layer "F.Cu") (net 2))
 (segment (start 122.199416 69.94) (end 122.199416 70.46) (width 0.5) (layer "F.Cu") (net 2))
 (segment (start 123.8 66.708636) (end 123.8 66.518477) (width 0.4) (layer "F.Cu") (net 2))
 (segment (start 120.158416 72.501) (end 104.620416 72.501) (width 0.4) (layer "F.Cu") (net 2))
 (segment (start 129.8 50.8) (end 129 50) (width 0.4) (layer "F.Cu") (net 2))
 (segment (start 102.559416 70.61) (end 102.559416 70.44) (width 0.4) (layer "F.Cu") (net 2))
 (segment (start 123.799 66.709636) (end 123.8 66.708636) (width 0.4) (layer "F.Cu") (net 2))
 (segment (start 129.8 55.808864) (end 129.8 50.8) (width 0.4) (layer "F.Cu") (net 2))
 (segment (start 122.199416 70.46) (end 120.158416 72.501) (width 0.4) (layer "F.Cu") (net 2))
 (segment (start 104.620416 72.501) (end 102.559416 70.44) (width 0.4) (layer "F.Cu") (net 2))
 (segment (start 127 56.4) (end 129.208864 56.4) (width 0.4) (layer "F.Cu") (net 2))
 (segment (start 129 50) (end 127.6 50) (width 0.4) (layer "F.Cu") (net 2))
 (segment (start 102.659416 70.51) (end 102.559416 70.61) (width 0.4) (layer "F.Cu") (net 2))
 (segment (start 126.099 57.301) (end 127 56.4) (width 0.4) (layer "F.Cu") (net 2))
 (segment (start 107.209416 59.48) (end 107.209416 58.290584) (width 0.4) (layer "F.Cu") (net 7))
 (segment (start 110.2 56.9) (end 115.881348 51.218652) (width 0.4) (layer "F.Cu") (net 7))
 (segment (start 116.99 48.01) (end 118.4 48.01) (width 0.4) (layer "F.Cu") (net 7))
 (segment (start 115.881348 51.218652) (end 115.881348 49.118652) (width 0.4) (layer "F.Cu") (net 7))
 (segment (start 117.769416 48.01) (end 117.769416 48.171155) (width 0.4) (layer "F.Cu") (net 7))
 (segment (start 107.209416 58.290584) (end 108.6 56.9) (width 0.4) (layer "F.Cu") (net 7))
 (segment (start 108.6 56.9) (end 110.2 56.9) (width 0.4) (layer "F.Cu") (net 7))
 (segment (start 115.881348 49.118652) (end 116.99 48.01) (width 0.4) (layer "F.Cu") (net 7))
 (segment (start 116.8 51.9) (end 109.749416 58.950584) (width 0.4) (layer "F.Cu") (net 8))
 (segment (start 109.749416 58.950584) (end 109.749416 59.48) (width 0.4) (layer "F.Cu") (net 8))
 (segment (start 116.8 50.5) (end 116.8 51.9) (width 0.4) (layer "F.Cu") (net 8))
 (segment (start 118.4 50.01) (end 117.29 50.01) (width 0.4) (layer "F.Cu") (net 8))
 (segment (start 117.29 50.01) (end 116.8 50.5) (width 0.4) (layer "F.Cu") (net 8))
 (segment (start 109.779416 58.25) (end 109.726186 58.30323) (width 0.2) (layer "F.Cu") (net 8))
 (segment (start 112.299416 58.22) (end 112.290501 58.228915) (width 0.2) (layer "F.Cu") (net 9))
 (segment (start 112.289416 57.910584) (end 118.19 52.01) (width 0.4) (layer "F.Cu") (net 9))
 (segment (start 112.289416 59.48) (end 112.289416 57.910584) (width 0.4) (layer "F.Cu") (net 9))
 (segment (start 118.19 52.01) (end 118.4 52.01) (width 0.4) (layer "F.Cu") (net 9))
 (segment (start 118.4 54.01) (end 117.69 54.01) (width 0.4) (layer "F.Cu") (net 10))
 (segment (start 117.69 54.01) (end 114.829416 56.870584) (width 0.4) (layer "F.Cu") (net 10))
 (segment (start 114.839416 58.27) (end 114.819416 58.29) (width 0.2) (layer "F.Cu") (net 10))
 (segment (start 114.829416 56.870584) (end 114.829416 59.48) (width 0.4) (layer "F.Cu") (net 10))
 (segment (start 123.958 55.138909) (end 123.457 54.637909) (width 0.4) (layer "F.Cu") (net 12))
 (segment (start 123.457 49.887) (end 121.58 48.01) (width 0.4) (layer "F.Cu") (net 12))
 (segment (start 125.462416 64.006117) (end 125.462416 57.4133) (width 0.4) (layer "F.Cu") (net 12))
 (segment (start 122.199416 67.96) (end 122.199416 67.269119) (width 0.4) (layer "F.Cu") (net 12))
 (segment (start 122.199416 67.269119) (end 125.462416 64.006117) (width 0.4) (layer "F.Cu") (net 12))
 (segment (start 123.958 55.908884) (end 123.958 55.138909) (width 0.4) (layer "F.Cu") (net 12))
 (segment (start 125.462416 57.4133) (end 123.958 55.908884) (width 0.4) (layer "F.Cu") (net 12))
 (segment (start 123.457 54.637909) (end 123.457 49.887) (width 0.4) (layer "F.Cu") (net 12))
 (segment (start 122.217395 66.401196) (end 124.861416 63.757175) (width 0.4) (layer "F.Cu") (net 11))
 (segment (start 122.856 54.886851) (end 122.856 51.286) (width 0.4) (layer "F.Cu") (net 11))
 (segment (start 107.679 71.879) (end 115.921 71.879) (width 0.4) (layer "F.Cu") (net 11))
 (segment (start 122.856 51.286) (end 121.58 50.01) (width 0.4) (layer "F.Cu") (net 11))
 (segment (start 115.921 71.879) (end 121.398804 66.401196) (width 0.4) (layer "F.Cu") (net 11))
 (segment (start 103.74 67.94) (end 107.679 71.879) (width 0.4) (layer "F.Cu") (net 11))
 (segment (start 124.861416 57.662242) (end 123.357 56.157826) (width 0.4) (layer "F.Cu") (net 11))
 (segment (start 121.398804 66.401196) (end 122.217395 66.401196) (width 0.4) (layer "F.Cu") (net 11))
 (segment (start 123.357 55.387851) (end 122.856 54.886851) (width 0.4) (layer "F.Cu") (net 11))
 (segment (start 123.357 56.157826) (end 123.357 55.387851) (width 0.4) (layer "F.Cu") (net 11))
 (segment (start 124.861416 63.757175) (end 124.861416 57.662242) (width 0.4) (layer "F.Cu") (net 11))
 (segment (start 102.559416 67.94) (end 103.74 67.94) (width 0.4) (layer "F.Cu") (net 11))
 (segment (start 120.2 55.672083) (end 120.813083 55.059) (width 0.3) (layer "F.Cu") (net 13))
 (segment (start 120.2 56.8) (end 120.2 55.672083) (width 0.3) (layer "F.Cu") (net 13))
 (segment (start 118.4 58.01) (end 118.99 58.01) (width 0.3) (layer "F.Cu") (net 13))
 (segment (start 118.99 58.01) (end 120.2 56.8) (width 0.3) (layer "F.Cu") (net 13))
 (segment (start 122.806 56.386058) (end 124.310416 57.890474) (width 0.3) (layer "F.Cu") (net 13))
 (segment (start 122.806 55.616083) (end 122.806 56.386058) (width 0.3) (layer "F.Cu") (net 13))
 (segment (start 108.728 71.328) (end 107.869416 70.469416) (width 0.3) (layer "F.Cu") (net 13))
 (segment (start 107.869416 70.469416) (end 107.869416 69) (width 0.3) (layer "F.Cu") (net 13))
 (segment (start 121.170572 65.850196) (end 115.692768 71.328) (width 0.3) (layer "F.Cu") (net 13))
 (segment (start 124.310416 57.890474) (end 124.310416 63.528944) (width 0.3) (layer "F.Cu") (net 13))
 (segment (start 115.692768 71.328) (end 108.728 71.328) (width 0.3) (layer "F.Cu") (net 13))
 (segment (start 121.989164 65.850196) (end 121.170572 65.850196) (width 0.3) (layer "F.Cu") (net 13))
 (segment (start 107.869416 69.51) (end 107.869416 69) (width 0.3) (layer "F.Cu") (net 13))
 (segment (start 120.813083 55.059) (end 122.248917 55.059) (width 0.3) (layer "F.Cu") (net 13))
 (segment (start 122.248917 55.059) (end 122.806 55.616083) (width 0.3) (layer "F.Cu") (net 13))
 (segment (start 124.310416 63.528944) (end 121.989164 65.850196) (width 0.3) (layer "F.Cu") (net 13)))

